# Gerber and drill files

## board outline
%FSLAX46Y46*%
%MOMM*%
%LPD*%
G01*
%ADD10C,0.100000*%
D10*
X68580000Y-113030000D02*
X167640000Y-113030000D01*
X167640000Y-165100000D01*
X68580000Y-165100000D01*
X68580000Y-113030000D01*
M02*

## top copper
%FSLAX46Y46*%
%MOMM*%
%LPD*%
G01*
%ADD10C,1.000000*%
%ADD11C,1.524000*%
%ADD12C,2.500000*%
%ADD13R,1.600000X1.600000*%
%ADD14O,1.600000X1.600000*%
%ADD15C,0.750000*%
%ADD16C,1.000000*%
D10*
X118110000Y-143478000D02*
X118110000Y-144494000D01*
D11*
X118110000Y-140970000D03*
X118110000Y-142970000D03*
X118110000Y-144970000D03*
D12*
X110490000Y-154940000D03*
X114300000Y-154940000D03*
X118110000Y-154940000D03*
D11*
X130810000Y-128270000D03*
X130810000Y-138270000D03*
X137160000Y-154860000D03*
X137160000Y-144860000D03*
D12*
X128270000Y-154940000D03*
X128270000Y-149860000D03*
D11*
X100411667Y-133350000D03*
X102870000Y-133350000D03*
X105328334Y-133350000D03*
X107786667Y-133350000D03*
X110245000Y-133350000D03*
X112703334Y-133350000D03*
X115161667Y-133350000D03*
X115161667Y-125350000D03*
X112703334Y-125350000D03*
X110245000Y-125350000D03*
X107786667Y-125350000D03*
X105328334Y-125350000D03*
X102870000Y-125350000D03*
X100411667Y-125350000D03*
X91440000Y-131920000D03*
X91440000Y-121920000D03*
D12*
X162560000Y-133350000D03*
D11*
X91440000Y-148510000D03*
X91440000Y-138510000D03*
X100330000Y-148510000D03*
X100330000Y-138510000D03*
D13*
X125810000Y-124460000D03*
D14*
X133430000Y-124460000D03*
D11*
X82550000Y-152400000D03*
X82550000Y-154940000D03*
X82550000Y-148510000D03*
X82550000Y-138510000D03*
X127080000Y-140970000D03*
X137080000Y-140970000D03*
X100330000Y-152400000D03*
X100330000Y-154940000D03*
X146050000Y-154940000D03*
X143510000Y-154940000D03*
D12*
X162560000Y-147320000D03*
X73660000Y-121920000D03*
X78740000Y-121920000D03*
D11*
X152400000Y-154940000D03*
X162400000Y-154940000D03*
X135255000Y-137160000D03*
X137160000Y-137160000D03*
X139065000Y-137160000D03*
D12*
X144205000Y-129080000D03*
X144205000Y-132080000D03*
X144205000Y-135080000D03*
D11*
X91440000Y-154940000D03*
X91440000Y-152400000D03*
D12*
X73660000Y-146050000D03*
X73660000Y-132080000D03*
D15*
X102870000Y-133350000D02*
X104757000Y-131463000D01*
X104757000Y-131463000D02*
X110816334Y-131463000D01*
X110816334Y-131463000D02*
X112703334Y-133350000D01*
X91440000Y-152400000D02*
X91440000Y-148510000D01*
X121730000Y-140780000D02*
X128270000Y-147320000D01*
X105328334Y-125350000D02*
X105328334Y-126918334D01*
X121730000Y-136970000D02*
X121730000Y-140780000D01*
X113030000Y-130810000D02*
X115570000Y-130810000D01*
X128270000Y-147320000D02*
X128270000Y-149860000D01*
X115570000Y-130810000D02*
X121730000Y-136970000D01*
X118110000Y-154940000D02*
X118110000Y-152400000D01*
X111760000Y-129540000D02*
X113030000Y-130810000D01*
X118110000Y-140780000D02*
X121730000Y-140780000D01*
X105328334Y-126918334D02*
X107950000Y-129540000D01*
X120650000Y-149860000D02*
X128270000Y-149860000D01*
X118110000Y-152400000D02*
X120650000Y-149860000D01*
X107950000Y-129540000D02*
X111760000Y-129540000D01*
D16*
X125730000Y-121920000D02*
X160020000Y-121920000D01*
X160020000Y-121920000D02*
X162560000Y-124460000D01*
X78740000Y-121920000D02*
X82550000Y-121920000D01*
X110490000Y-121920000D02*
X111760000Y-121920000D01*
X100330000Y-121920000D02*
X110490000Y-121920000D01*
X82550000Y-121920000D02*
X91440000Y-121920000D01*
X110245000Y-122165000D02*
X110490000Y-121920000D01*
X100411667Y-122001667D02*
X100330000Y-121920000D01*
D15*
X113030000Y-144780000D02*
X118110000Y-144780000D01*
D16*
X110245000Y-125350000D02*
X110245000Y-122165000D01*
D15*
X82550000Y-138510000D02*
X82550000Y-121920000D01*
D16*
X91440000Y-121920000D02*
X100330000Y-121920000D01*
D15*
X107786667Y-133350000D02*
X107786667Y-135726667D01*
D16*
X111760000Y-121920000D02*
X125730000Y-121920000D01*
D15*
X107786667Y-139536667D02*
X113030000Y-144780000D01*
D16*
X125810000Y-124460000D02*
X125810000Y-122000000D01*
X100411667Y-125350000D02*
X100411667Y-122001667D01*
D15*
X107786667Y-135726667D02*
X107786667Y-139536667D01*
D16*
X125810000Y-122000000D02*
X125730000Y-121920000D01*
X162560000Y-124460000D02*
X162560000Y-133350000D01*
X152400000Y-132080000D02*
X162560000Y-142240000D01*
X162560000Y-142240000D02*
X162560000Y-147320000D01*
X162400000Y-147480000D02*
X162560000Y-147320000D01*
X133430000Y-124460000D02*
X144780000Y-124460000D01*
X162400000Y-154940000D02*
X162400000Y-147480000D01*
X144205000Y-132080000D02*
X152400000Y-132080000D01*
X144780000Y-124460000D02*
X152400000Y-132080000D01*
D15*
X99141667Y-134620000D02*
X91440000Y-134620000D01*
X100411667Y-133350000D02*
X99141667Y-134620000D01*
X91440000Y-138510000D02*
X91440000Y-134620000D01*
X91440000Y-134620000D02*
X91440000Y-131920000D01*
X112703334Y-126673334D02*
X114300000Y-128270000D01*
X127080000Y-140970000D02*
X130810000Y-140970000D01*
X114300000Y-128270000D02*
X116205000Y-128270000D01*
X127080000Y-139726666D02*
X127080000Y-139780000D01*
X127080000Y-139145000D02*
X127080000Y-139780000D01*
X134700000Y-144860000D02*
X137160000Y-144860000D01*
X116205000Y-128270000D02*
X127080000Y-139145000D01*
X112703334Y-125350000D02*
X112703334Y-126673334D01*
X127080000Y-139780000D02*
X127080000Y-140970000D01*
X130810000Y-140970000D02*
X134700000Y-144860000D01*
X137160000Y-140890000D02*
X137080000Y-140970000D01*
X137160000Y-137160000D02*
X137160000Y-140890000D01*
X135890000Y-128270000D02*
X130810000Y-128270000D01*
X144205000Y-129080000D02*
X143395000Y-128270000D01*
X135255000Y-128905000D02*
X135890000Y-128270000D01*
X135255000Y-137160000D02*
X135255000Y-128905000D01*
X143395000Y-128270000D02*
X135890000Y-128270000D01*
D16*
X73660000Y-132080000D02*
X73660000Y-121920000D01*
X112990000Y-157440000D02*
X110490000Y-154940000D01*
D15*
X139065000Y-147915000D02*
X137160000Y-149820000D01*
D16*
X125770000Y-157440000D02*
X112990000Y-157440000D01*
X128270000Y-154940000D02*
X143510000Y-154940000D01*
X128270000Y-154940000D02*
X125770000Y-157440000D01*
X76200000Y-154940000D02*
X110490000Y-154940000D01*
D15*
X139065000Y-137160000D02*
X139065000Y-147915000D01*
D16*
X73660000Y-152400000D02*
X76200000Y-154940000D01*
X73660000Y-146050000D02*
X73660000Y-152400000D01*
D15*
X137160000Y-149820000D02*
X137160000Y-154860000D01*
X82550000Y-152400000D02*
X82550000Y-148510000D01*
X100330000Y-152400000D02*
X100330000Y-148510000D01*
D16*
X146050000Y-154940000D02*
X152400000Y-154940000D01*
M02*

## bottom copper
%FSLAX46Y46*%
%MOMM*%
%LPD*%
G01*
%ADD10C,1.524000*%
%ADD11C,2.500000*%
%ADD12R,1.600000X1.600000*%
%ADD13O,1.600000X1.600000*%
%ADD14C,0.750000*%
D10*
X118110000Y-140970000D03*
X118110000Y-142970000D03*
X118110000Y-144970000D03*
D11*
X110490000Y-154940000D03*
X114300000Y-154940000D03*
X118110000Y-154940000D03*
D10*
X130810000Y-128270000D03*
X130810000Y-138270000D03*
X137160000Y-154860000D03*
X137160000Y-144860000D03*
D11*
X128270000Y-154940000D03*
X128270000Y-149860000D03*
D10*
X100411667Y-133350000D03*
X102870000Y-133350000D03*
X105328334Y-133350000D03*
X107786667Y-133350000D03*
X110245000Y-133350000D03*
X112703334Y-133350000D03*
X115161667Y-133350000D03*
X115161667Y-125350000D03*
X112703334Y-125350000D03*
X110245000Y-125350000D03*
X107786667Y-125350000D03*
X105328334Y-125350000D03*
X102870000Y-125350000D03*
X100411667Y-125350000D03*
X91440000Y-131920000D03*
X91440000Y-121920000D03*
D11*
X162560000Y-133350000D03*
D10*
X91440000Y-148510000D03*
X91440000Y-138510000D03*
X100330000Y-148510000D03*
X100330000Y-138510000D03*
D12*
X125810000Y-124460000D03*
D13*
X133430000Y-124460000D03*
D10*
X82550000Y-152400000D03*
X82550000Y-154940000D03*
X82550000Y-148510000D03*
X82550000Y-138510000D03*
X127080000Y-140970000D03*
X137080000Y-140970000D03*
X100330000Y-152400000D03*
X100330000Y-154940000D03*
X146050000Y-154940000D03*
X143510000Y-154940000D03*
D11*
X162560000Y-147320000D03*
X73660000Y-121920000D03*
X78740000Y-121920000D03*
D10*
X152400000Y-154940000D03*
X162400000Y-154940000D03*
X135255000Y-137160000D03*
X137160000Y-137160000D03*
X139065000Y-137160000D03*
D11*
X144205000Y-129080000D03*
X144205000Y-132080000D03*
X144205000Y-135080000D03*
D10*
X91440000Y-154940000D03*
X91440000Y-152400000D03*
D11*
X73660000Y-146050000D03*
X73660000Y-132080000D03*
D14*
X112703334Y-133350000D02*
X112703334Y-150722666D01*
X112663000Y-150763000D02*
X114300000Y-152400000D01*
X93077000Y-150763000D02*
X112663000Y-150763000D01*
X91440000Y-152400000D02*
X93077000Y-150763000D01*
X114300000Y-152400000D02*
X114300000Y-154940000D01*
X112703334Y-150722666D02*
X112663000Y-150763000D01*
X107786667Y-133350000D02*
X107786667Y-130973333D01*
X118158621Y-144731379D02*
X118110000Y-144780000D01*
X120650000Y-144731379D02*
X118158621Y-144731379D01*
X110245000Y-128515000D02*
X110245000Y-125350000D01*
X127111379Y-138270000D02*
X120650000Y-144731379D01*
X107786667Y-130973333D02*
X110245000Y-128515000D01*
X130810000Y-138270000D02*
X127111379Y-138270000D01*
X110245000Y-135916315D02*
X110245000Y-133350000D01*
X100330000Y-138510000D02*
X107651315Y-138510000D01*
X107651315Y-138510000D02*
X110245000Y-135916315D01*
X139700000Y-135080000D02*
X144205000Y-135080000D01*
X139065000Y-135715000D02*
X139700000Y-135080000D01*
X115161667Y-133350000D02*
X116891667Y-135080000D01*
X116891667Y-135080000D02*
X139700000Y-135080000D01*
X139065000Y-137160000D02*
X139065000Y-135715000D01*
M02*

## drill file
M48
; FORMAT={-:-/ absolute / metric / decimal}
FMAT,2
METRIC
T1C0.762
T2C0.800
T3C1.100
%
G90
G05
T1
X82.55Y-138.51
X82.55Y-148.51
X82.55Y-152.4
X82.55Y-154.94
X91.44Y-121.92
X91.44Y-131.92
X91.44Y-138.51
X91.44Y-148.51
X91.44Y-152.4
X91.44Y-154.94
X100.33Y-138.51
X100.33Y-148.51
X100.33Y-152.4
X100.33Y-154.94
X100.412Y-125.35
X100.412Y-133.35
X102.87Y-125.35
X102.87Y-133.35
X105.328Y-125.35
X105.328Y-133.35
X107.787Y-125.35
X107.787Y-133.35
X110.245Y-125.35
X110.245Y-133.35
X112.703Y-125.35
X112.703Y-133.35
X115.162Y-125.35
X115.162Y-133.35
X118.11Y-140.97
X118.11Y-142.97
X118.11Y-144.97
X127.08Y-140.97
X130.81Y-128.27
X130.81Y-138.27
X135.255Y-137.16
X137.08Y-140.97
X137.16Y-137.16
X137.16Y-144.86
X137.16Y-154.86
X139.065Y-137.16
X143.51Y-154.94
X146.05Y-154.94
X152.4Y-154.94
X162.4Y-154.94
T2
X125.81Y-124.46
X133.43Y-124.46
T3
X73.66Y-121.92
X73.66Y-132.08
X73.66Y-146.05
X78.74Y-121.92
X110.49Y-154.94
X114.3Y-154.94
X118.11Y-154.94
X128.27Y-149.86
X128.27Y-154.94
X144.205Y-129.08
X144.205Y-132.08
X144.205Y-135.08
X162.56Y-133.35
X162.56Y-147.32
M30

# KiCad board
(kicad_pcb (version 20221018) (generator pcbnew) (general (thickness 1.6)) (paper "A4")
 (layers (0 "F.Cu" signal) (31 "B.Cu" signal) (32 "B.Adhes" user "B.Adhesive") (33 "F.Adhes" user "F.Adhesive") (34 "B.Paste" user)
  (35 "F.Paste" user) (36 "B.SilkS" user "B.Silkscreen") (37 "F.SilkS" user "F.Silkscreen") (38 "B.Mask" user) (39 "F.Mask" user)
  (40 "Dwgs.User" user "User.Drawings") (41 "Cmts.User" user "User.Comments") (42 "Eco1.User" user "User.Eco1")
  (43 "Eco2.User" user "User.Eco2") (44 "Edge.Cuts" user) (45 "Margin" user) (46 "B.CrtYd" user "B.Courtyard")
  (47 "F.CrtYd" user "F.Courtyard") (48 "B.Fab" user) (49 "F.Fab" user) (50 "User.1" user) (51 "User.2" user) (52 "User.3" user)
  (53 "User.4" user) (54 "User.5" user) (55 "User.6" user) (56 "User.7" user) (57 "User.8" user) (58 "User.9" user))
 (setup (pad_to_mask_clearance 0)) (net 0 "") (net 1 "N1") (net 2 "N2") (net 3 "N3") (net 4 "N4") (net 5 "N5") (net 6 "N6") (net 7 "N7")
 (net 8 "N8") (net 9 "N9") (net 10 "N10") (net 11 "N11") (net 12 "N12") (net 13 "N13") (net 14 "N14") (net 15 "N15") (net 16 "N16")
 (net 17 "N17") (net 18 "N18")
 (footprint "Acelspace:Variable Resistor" (layer "F.Cu") (at 118.11 142.97 -90)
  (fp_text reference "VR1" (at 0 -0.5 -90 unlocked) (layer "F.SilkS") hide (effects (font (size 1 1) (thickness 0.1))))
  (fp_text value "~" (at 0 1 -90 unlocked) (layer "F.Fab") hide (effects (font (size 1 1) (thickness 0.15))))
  (fp_line (start 0.508 0) (end 1.524 0) (stroke (width 1) (type default)) (layer "F.Cu"))
  (pad "1" thru_hole circle (at -2 0 270) (size 1.524 1.524) (drill 0.762) (layers "*.Cu" "*.Mask") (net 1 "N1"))
  (pad "2" thru_hole circle (at 0 0 270) (size 1.524 1.524) (drill 0.762) (layers "*.Cu" "*.Mask"))
  (pad "3" thru_hole circle (at 2 0 270) (size 1.524 1.524) (drill 0.762) (layers "*.Cu" "*.Mask") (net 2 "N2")))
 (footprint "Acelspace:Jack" (layer "F.Cu") (at 114.3 154.94)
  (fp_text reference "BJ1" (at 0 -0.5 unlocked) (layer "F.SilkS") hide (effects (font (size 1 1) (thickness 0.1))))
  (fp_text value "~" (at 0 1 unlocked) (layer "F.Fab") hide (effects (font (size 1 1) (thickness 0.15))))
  (pad "1" thru_hole circle (at -3.81 0) (size 2.5 2.5) (drill 1.1) (layers "*.Cu" "*.Mask") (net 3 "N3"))
  (pad "2" thru_hole circle (at 0 0) (size 2.5 2.5) (drill 1.1) (layers "*.Cu" "*.Mask") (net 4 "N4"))
  (pad "3" thru_hole circle (at 3.81 0) (size 2.5 2.5) (drill 1.1) (layers "*.Cu" "*.Mask") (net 1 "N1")))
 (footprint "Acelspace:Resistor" (layer "F.Cu") (at 130.81 133.27 -90)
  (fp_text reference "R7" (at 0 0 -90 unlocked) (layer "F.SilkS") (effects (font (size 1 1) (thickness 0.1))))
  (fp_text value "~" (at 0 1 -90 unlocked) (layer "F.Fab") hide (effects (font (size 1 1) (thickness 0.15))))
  (pad "1" thru_hole circle (at -5 0 270) (size 1.524 1.524) (drill 0.762) (layers "*.Cu" "*.Mask") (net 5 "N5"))
  (pad "2" thru_hole circle (at 5 0 270) (size 1.524 1.524) (drill 0.762) (layers "*.Cu" "*.Mask") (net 2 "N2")))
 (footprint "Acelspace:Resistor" (layer "F.Cu") (at 137.16 149.86 90)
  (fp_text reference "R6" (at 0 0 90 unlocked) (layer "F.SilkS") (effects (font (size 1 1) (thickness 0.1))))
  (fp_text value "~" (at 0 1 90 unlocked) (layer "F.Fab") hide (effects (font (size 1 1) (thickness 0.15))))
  (pad "1" thru_hole circle (at -5 0 90) (size 1.524 1.524) (drill 0.762) (layers "*.Cu" "*.Mask") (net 3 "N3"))
  (pad "2" thru_hole circle (at 5 0 90) (size 1.524 1.524) (drill 0.762) (layers "*.Cu" "*.Mask") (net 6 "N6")))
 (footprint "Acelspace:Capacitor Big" (layer "F.Cu") (at 128.27 152.4 180)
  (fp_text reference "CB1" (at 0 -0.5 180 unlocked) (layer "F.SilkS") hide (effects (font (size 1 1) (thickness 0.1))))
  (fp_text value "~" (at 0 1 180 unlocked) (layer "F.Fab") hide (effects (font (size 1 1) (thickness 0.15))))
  (pad "1" thru_hole circle (at 0 -2.54 180) (size 2.5 2.5) (drill 1.1) (layers "*.Cu" "*.Mask") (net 3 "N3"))
  (pad "2" thru_hole circle (at 0 2.54 180) (size 2.5 2.5) (drill 1.1) (layers "*.Cu" "*.Mask") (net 1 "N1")))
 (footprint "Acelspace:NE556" (layer "F.Cu") (at 107.786667 129.35 -90)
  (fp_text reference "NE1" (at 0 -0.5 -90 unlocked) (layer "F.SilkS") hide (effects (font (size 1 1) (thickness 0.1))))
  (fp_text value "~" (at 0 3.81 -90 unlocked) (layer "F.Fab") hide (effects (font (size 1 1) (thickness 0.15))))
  (pad "1" thru_hole circle (at 4 7.375 270) (size 1.524 1.524) (drill 0.762) (layers "*.Cu" "*.Mask") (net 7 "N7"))
  (pad "2" thru_hole circle (at 4 4.916667 270) (size 1.524 1.524) (drill 0.762) (layers "*.Cu" "*.Mask") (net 4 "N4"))
  (pad "3" thru_hole circle (at 4 2.458333 270) (size 1.524 1.524) (drill 0.762) (layers "*.Cu" "*.Mask") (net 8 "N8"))
  (pad "4" thru_hole circle (at 4 0 270) (size 1.524 1.524) (drill 0.762) (layers "*.Cu" "*.Mask") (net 2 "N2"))
  (pad "5" thru_hole circle (at 4 -2.458333 270) (size 1.524 1.524) (drill 0.762) (layers "*.Cu" "*.Mask") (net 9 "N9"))
  (pad "6" thru_hole circle (at 4 -4.916667 270) (size 1.524 1.524) (drill 0.762) (layers "*.Cu" "*.Mask") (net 4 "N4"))
  (pad "7" thru_hole circle (at 4 -7.375 270) (size 1.524 1.524) (drill 0.762) (layers "*.Cu" "*.Mask") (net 3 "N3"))
  (pad "8" thru_hole circle (at -4 -7.375 270) (size 1.524 1.524) (drill 0.762) (layers "*.Cu" "*.Mask") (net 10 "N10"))
  (pad "9" thru_hole circle (at -4 -4.916667 270) (size 1.524 1.524) (drill 0.762) (layers "*.Cu" "*.Mask") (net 6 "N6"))
  (pad "10" thru_hole circle (at -4 -2.458333 270) (size 1.524 1.524) (drill 0.762) (layers "*.Cu" "*.Mask") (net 2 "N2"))
  (pad "11" thru_hole circle (at -4 0 270) (size 1.524 1.524) (drill 0.762) (layers "*.Cu" "*.Mask") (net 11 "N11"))
  (pad "12" thru_hole circle (at -4 2.458333 270) (size 1.524 1.524) (drill 0.762) (layers "*.Cu" "*.Mask") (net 1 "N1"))
  (pad "13" thru_hole circle (at -4 4.916667 270) (size 1.524 1.524) (drill 0.762) (layers "*.Cu" "*.Mask") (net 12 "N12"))
  (pad "14" thru_hole circle (at -4 7.375 270) (size 1.524 1.524) (drill 0.762) (layers "*.Cu" "*.Mask") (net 2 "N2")))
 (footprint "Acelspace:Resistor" (layer "F.Cu") (at 91.44 126.92 90)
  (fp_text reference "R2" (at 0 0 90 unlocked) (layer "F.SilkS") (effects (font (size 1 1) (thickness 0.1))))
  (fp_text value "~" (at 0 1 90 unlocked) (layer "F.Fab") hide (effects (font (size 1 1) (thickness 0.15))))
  (pad "1" thru_hole circle (at -5 0 90) (size 1.524 1.524) (drill 0.762) (layers "*.Cu" "*.Mask") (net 7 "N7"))
  (pad "2" thru_hole circle (at 5 0 90) (size 1.524 1.524) (drill 0.762) (layers "*.Cu" "*.Mask") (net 2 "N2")))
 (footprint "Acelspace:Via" (layer "F.Cu") (at 162.56 133.35)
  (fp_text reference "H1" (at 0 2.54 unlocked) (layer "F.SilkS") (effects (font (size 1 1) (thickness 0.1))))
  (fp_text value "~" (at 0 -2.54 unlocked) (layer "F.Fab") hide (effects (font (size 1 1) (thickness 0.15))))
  (pad "1" thru_hole circle (at 0 0) (size 2.5 2.5) (drill 1.1) (layers "*.Cu" "*.Mask") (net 2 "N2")))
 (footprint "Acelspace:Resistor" (layer "F.Cu") (at 91.44 143.51 90)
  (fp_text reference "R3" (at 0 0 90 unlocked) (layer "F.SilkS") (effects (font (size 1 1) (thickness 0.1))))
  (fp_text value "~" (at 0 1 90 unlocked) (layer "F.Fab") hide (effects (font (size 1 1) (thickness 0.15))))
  (pad "1" thru_hole circle (at -5 0 90) (size 1.524 1.524) (drill 0.762) (layers "*.Cu" "*.Mask") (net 4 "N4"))
  (pad "2" thru_hole circle (at 5 0 90) (size 1.524 1.524) (drill 0.762) (layers "*.Cu" "*.Mask") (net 7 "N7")))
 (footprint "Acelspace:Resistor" (layer "F.Cu") (at 100.33 143.51 90)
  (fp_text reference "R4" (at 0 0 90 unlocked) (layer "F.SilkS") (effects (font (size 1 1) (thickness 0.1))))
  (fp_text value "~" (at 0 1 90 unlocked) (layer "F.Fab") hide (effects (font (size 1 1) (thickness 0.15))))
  (pad "1" thru_hole circle (at -5 0 90) (size 1.524 1.524) (drill 0.762) (layers "*.Cu" "*.Mask") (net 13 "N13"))
  (pad "2" thru_hole circle (at 5 0 90) (size 1.524 1.524) (drill 0.762) (layers "*.Cu" "*.Mask") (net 9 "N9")))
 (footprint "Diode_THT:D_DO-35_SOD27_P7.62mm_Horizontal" (layer "F.Cu") (at 125.81 124.46)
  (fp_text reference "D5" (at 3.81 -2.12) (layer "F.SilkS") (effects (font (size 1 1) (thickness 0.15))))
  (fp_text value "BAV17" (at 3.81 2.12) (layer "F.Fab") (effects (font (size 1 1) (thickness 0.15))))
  (pad "1" thru_hole rect (at 0 0) (size 1.6 1.6) (drill 0.8) (layers "*.Cu" "*.Mask") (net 2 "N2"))
  (pad "2" thru_hole oval (at 7.62 0) (size 1.6 1.6) (drill 0.8) (layers "*.Cu" "*.Mask") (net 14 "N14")))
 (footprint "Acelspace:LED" (layer "F.Cu") (at 82.55 153.67 90)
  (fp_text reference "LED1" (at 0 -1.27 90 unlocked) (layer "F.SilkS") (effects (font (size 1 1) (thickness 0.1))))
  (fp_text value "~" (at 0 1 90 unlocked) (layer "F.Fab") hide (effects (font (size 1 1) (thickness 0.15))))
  (pad "1" thru_hole circle (at 1.27 0 90) (size 1.524 1.524) (drill 0.762) (layers "*.Cu" "*.Mask") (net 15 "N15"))
  (pad "2" thru_hole circle (at -1.27 0 90) (size 1.524 1.524) (drill 0.762) (layers "*.Cu" "*.Mask") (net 3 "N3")))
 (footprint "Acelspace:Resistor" (layer "F.Cu") (at 82.55 143.51 90)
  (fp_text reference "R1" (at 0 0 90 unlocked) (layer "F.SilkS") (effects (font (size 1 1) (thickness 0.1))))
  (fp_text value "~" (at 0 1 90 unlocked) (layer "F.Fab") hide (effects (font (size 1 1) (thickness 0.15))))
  (pad "1" thru_hole circle (at -5 0 90) (size 1.524 1.524) (drill 0.762) (layers "*.Cu" "*.Mask") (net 15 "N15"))
  (pad "2" thru_hole circle (at 5 0 90) (size 1.524 1.524) (drill 0.762) (layers "*.Cu" "*.Mask") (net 2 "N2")))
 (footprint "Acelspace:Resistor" (layer "F.Cu") (at 132.08 140.97)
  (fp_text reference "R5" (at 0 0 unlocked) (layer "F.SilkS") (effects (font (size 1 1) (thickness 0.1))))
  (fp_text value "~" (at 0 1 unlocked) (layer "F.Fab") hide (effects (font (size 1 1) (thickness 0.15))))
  (pad "1" thru_hole circle (at -5 0) (size 1.524 1.524) (drill 0.762) (layers "*.Cu" "*.Mask") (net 6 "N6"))
  (pad "2" thru_hole circle (at 5 0) (size 1.524 1.524) (drill 0.762) (layers "*.Cu" "*.Mask") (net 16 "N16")))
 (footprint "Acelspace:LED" (layer "F.Cu") (at 100.33 153.67 90)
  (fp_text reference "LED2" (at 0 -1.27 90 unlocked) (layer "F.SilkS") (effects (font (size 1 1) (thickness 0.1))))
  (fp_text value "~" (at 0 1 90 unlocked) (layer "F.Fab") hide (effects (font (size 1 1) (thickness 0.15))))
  (pad "1" thru_hole circle (at 1.27 0 90) (size 1.524 1.524) (drill 0.762) (layers "*.Cu" "*.Mask") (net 13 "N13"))
  (pad "2" thru_hole circle (at -1.27 0 90) (size 1.524 1.524) (drill 0.762) (layers "*.Cu" "*.Mask") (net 3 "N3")))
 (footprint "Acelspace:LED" (layer "F.Cu") (at 144.78 154.94)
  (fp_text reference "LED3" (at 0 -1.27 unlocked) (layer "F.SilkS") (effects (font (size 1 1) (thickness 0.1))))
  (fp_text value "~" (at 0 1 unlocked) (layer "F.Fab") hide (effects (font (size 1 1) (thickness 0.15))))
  (pad "1" thru_hole circle (at 1.27 0) (size 1.524 1.524) (drill 0.762) (layers "*.Cu" "*.Mask") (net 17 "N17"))
  (pad "2" thru_hole circle (at -1.27 0) (size 1.524 1.524) (drill 0.762) (layers "*.Cu" "*.Mask") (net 3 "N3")))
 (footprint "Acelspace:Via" (layer "F.Cu") (at 162.56 147.32)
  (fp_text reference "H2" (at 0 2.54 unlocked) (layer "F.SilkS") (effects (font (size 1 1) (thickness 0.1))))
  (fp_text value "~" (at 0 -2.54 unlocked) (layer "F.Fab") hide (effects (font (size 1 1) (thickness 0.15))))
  (pad "1" thru_hole circle (at 0 0) (size 2.5 2.5) (drill 1.1) (layers "*.Cu" "*.Mask") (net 14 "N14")))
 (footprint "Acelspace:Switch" (layer "F.Cu") (at 76.2 121.92)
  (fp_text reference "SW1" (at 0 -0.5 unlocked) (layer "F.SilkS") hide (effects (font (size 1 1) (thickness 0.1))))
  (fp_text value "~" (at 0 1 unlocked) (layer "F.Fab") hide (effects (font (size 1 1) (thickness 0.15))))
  (pad "1" thru_hole circle (at -2.54 0) (size 2.5 2.5) (drill 1.1) (layers "*.Cu" "*.Mask") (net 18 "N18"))
  (pad "2" thru_hole circle (at 2.54 0) (size 2.5 2.5) (drill 1.1) (layers "*.Cu" "*.Mask") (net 2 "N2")))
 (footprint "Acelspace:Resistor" (layer "F.Cu") (at 157.4 154.94)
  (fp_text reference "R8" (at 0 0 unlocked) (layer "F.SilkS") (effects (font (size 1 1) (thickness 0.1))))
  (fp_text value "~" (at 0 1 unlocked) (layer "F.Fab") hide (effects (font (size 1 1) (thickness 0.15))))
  (pad "1" thru_hole circle (at -5 0) (size 1.524 1.524) (drill 0.762) (layers "*.Cu" "*.Mask") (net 17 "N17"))
  (pad "2" thru_hole circle (at 5 0) (size 1.524 1.524) (drill 0.762) (layers "*.Cu" "*.Mask") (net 14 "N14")))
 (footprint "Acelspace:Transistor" (layer "F.Cu") (at 137.16 137.16)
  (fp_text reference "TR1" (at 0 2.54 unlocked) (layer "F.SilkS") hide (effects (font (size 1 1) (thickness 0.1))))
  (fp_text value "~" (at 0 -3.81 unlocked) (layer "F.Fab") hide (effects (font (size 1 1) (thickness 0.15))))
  (pad "1" thru_hole circle (at -1.905 0) (size 1.524 1.524) (drill 0.762) (layers "*.Cu" "*.Mask") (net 5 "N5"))
  (pad "2" thru_hole circle (at 0 0) (size 1.524 1.524) (drill 0.762) (layers "*.Cu" "*.Mask") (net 16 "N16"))
  (pad "3" thru_hole circle (at 1.905 0) (size 1.524 1.524) (drill 0.762) (layers "*.Cu" "*.Mask") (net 3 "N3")))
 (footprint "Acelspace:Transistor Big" (layer "F.Cu") (at 144.205 132.08 -90)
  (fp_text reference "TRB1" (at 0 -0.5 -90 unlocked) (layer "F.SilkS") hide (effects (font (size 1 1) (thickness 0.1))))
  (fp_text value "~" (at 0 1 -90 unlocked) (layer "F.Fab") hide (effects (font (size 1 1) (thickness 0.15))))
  (pad "1" thru_hole circle (at -3 0 270) (size 2.5 2.5) (drill 1.1) (layers "*.Cu" "*.Mask") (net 5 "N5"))
  (pad "2" thru_hole circle (at 0 0 270) (size 2.5 2.5) (drill 1.1) (layers "*.Cu" "*.Mask") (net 14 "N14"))
  (pad "3" thru_hole circle (at 3 0 270) (size 2.5 2.5) (drill 1.1) (layers "*.Cu" "*.Mask") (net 3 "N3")))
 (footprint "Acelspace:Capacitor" (layer "F.Cu") (at 91.44 153.67 180)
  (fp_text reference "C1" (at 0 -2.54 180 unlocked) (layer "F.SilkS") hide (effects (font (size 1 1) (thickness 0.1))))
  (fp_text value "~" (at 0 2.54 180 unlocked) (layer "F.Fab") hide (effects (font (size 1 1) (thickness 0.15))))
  (pad "1" thru_hole circle (at 0 -1.27 180) (size 1.524 1.524) (drill 0.762) (layers "*.Cu" "*.Mask") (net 3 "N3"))
  (pad "2" thru_hole circle (at 0 1.27 180) (size 1.524 1.524) (drill 0.762) (layers "*.Cu" "*.Mask") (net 4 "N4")))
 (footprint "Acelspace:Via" (layer "F.Cu") (at 73.66 146.05)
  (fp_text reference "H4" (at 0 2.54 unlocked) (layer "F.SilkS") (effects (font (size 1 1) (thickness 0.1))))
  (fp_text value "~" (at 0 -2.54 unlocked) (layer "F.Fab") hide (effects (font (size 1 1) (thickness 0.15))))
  (pad "1" thru_hole circle (at 0 0) (size 2.5 2.5) (drill 1.1) (layers "*.Cu" "*.Mask") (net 3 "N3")))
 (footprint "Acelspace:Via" (layer "F.Cu") (at 73.66 132.08)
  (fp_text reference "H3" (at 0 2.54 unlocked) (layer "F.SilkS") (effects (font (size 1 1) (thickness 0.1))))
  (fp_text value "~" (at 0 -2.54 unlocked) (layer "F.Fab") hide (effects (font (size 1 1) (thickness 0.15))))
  (pad "1" thru_hole circle (at 0 0) (size 2.5 2.5) (drill 1.1) (layers "*.Cu" "*.Mask") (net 18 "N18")))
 (gr_rect (start 68.58 113.03) (end 167.64 165.1) (stroke (width 0.1) (type default)) (fill none) (layer "Edge.Cuts"))
 (segment (start 102.87 133.35) (end 104.757 131.463) (width 0.75) (layer "F.Cu") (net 4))
 (segment (start 104.757 131.463) (end 110.816334 131.463) (width 0.75) (layer "F.Cu") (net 4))
 (segment (start 110.816334 131.463) (end 112.703334 133.35) (width 0.75) (layer "F.Cu") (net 4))
 (segment (start 91.44 152.4) (end 91.44 148.51) (width 0.75) (layer "F.Cu") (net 4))
 (segment (start 112.703334 133.35) (end 112.703334 150.722666) (width 0.75) (layer "B.Cu") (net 4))
 (segment (start 112.663 150.763) (end 114.3 152.4) (width 0.75) (layer "B.Cu") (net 4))
 (segment (start 93.077 150.763) (end 112.663 150.763) (width 0.75) (layer "B.Cu") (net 4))
 (segment (start 91.44 152.4) (end 93.077 150.763) (width 0.75) (layer "B.Cu") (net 4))
 (segment (start 114.3 152.4) (end 114.3 154.94) (width 0.75) (layer "B.Cu") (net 4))
 (segment (start 112.703334 150.722666) (end 112.663 150.763) (width 0.75) (layer "B.Cu") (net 4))
 (segment (start 121.73 140.78) (end 128.27 147.32) (width 0.75) (layer "F.Cu") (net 1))
 (segment (start 105.328334 125.35) (end 105.328334 126.918334) (width 0.75) (layer "F.Cu") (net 1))
 (segment (start 121.73 136.97) (end 121.73 140.78) (width 0.75) (layer "F.Cu") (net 1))
 (segment (start 113.03 130.81) (end 115.57 130.81) (width 0.75) (layer "F.Cu") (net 1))
 (segment (start 128.27 147.32) (end 128.27 149.86) (width 0.75) (layer "F.Cu") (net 1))
 (segment (start 115.57 130.81) (end 121.73 136.97) (width 0.75) (layer "F.Cu") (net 1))
 (segment (start 118.11 154.94) (end 118.11 152.4) (width 0.75) (layer "F.Cu") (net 1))
 (segment (start 111.76 129.54) (end 113.03 130.81) (width 0.75) (layer "F.Cu") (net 1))
 (segment (start 118.11 140.78) (end 121.73 140.78) (width 0.75) (layer "F.Cu") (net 1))
 (segment (start 105.328334 126.918334) (end 107.95 129.54) (width 0.75) (layer "F.Cu") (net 1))
 (segment (start 120.65 149.86) (end 128.27 149.86) (width 0.75) (layer "F.Cu") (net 1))
 (segment (start 118.11 152.4) (end 120.65 149.86) (width 0.75) (layer "F.Cu") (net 1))
 (segment (start 107.95 129.54) (end 111.76 129.54) (width 0.75) (layer "F.Cu") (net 1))
 (segment (start 125.73 121.92) (end 160.02 121.92) (width 1) (layer "F.Cu") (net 2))
 (segment (start 160.02 121.92) (end 162.56 124.46) (width 1) (layer "F.Cu") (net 2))
 (segment (start 78.74 121.92) (end 82.55 121.92) (width 1) (layer "F.Cu") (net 2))
 (segment (start 110.49 121.92) (end 111.76 121.92) (width 1) (layer "F.Cu") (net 2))
 (segment (start 100.33 121.92) (end 110.49 121.92) (width 1) (layer "F.Cu") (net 2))
 (segment (start 82.55 121.92) (end 91.44 121.92) (width 1) (layer "F.Cu") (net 2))
 (segment (start 110.245 122.165) (end 110.49 121.92) (width 1) (layer "F.Cu") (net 2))
 (segment (start 100.411667 122.001667) (end 100.33 121.92) (width 1) (layer "F.Cu") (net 2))
 (segment (start 113.03 144.78) (end 118.11 144.78) (width 0.75) (layer "F.Cu") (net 2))
 (segment (start 110.245 125.35) (end 110.245 122.165) (width 1) (layer "F.Cu") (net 2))
 (segment (start 82.55 138.51) (end 82.55 121.92) (width 0.75) (layer "F.Cu") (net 2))
 (segment (start 91.44 121.92) (end 100.33 121.92) (width 1) (layer "F.Cu") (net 2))
 (segment (start 107.786667 133.35) (end 107.786667 135.726667) (width 0.75) (layer "F.Cu") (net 2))
 (segment (start 111.76 121.92) (end 125.73 121.92) (width 1) (layer "F.Cu") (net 2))
 (segment (start 107.786667 139.536667) (end 113.03 144.78) (width 0.75) (layer "F.Cu") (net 2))
 (segment (start 125.81 124.46) (end 125.81 122) (width 1) (layer "F.Cu") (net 2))
 (segment (start 100.411667 125.35) (end 100.411667 122.001667) (width 1) (layer "F.Cu") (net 2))
 (segment (start 107.786667 135.726667) (end 107.786667 139.536667) (width 0.75) (layer "F.Cu") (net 2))
 (segment (start 125.81 122) (end 125.73 121.92) (width 1) (layer "F.Cu") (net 2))
 (segment (start 162.56 124.46) (end 162.56 133.35) (width 1) (layer "F.Cu") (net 2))
 (segment (start 107.786667 133.35) (end 107.786667 130.973333) (width 0.75) (layer "B.Cu") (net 2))
 (segment (start 118.158621 144.731379) (end 118.11 144.78) (width 0.75) (layer "B.Cu") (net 2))
 (segment (start 120.65 144.731379) (end 118.158621 144.731379) (width 0.75) (layer "B.Cu") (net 2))
 (segment (start 110.245 128.515) (end 110.245 125.35) (width 0.75) (layer "B.Cu") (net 2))
 (segment (start 127.111379 138.27) (end 120.65 144.731379) (width 0.75) (layer "B.Cu") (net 2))
 (segment (start 107.786667 130.973333) (end 110.245 128.515) (width 0.75) (layer "B.Cu") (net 2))
 (segment (start 130.81 138.27) (end 127.111379 138.27) (width 0.75) (layer "B.Cu") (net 2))
 (segment (start 152.4 132.08) (end 162.56 142.24) (width 1) (layer "F.Cu") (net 14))
 (segment (start 162.56 142.24) (end 162.56 147.32) (width 1) (layer "F.Cu") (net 14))
 (segment (start 162.4 147.48) (end 162.56 147.32) (width 1) (layer "F.Cu") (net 14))
 (segment (start 133.43 124.46) (end 144.78 124.46) (width 1) (layer "F.Cu") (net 14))
 (segment (start 162.4 154.94) (end 162.4 147.48) (width 1) (layer "F.Cu") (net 14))
 (segment (start 144.205 132.08) (end 152.4 132.08) (width 1) (layer "F.Cu") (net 14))
 (segment (start 144.78 124.46) (end 152.4 132.08) (width 1) (layer "F.Cu") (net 14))
 (segment (start 99.141667 134.62) (end 91.44 134.62) (width 0.75) (layer "F.Cu") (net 7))
 (segment (start 100.411667 133.35) (end 99.141667 134.62) (width 0.75) (layer "F.Cu") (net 7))
 (segment (start 91.44 138.51) (end 91.44 134.62) (width 0.75) (layer "F.Cu") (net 7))
 (segment (start 91.44 134.62) (end 91.44 131.92) (width 0.75) (layer "F.Cu") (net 7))
 (segment (start 110.245 135.916315) (end 110.245 133.35) (width 0.75) (layer "B.Cu") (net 9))
 (segment (start 100.33 138.51) (end 107.651315 138.51) (width 0.75) (layer "B.Cu") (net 9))
 (segment (start 107.651315 138.51) (end 110.245 135.916315) (width 0.75) (layer "B.Cu") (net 9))
 (segment (start 112.703334 126.673334) (end 114.3 128.27) (width 0.75) (layer "F.Cu") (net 6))
 (segment (start 127.08 140.97) (end 130.81 140.97) (width 0.75) (layer "F.Cu") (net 6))
 (segment (start 114.3 128.27) (end 116.205 128.27) (width 0.75) (layer "F.Cu") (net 6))
 (segment (start 127.08 139.726666) (end 127.08 139.78) (width 0.75) (layer "F.Cu") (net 6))
 (segment (start 127.08 139.145) (end 127.08 139.78) (width 0.75) (layer "F.Cu") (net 6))
 (segment (start 134.7 144.86) (end 137.16 144.86) (width 0.75) (layer "F.Cu") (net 6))
 (segment (start 116.205 128.27) (end 127.08 139.145) (width 0.75) (layer "F.Cu") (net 6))
 (segment (start 112.703334 125.35) (end 112.703334 126.673334) (width 0.75) (layer "F.Cu") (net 6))
 (segment (start 127.08 139.78) (end 127.08 140.97) (width 0.75) (layer "F.Cu") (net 6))
 (segment (start 130.81 140.97) (end 134.7 144.86) (width 0.75) (layer "F.Cu") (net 6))
 (segment (start 137.16 140.89) (end 137.08 140.97) (width 0.75) (layer "F.Cu") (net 16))
 (segment (start 137.16 137.16) (end 137.16 140.89) (width 0.75) (layer "F.Cu") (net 16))
 (segment (start 135.89 128.27) (end 130.81 128.27) (width 0.75) (layer "F.Cu") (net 5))
 (segment (start 144.205 129.08) (end 143.395 128.27) (width 0.75) (layer "F.Cu") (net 5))
 (segment (start 135.255 128.905) (end 135.89 128.27) (width 0.75) (layer "F.Cu") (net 5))
 (segment (start 135.255 137.16) (end 135.255 128.905) (width 0.75) (layer "F.Cu") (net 5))
 (segment (start 143.395 128.27) (end 135.89 128.27) (width 0.75) (layer "F.Cu") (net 5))
 (segment (start 73.66 132.08) (end 73.66 121.92) (width 1) (layer "F.Cu") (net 18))
 (segment (start 112.99 157.44) (end 110.49 154.94) (width 1) (layer "F.Cu") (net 3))
 (segment (start 139.065 147.915) (end 137.16 149.82) (width 0.75) (layer "F.Cu") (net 3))
 (segment (start 125.77 157.44) (end 112.99 157.44) (width 1) (layer "F.Cu") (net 3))
 (segment (start 128.27 154.94) (end 143.51 154.94) (width 1) (layer "F.Cu") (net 3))
 (segment (start 128.27 154.94) (end 125.77 157.44) (width 1) (layer "F.Cu") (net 3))
 (segment (start 76.2 154.94) (end 110.49 154.94) (width 1) (layer "F.Cu") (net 3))
 (segment (start 139.065 137.16) (end 139.065 147.915) (width 0.75) (layer "F.Cu") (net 3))
 (segment (start 73.66 152.4) (end 76.2 154.94) (width 1) (layer "F.Cu") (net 3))
 (segment (start 73.66 146.05) (end 73.66 152.4) (width 1) (layer "F.Cu") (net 3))
 (segment (start 137.16 149.82) (end 137.16 154.86) (width 0.75) (layer "F.Cu") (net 3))
 (segment (start 139.7 135.08) (end 144.205 135.08) (width 0.75) (layer "B.Cu") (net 3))
 (segment (start 139.065 135.715) (end 139.7 135.08) (width 0.75) (layer "B.Cu") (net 3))
 (segment (start 115.161667 133.35) (end 116.891667 135.08) (width 0.75) (layer "B.Cu") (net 3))
 (segment (start 116.891667 135.08) (end 139.7 135.08) (width 0.75) (layer "B.Cu") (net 3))
 (segment (start 139.065 137.16) (end 139.065 135.715) (width 0.75) (layer "B.Cu") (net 3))
 (segment (start 82.55 152.4) (end 82.55 148.51) (width 0.75) (layer "F.Cu") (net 15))
 (segment (start 100.33 152.4) (end 100.33 148.51) (width 0.75) (layer "F.Cu") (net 13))
 (segment (start 146.05 154.94) (end 152.4 154.94) (width 1) (layer "F.Cu") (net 17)))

